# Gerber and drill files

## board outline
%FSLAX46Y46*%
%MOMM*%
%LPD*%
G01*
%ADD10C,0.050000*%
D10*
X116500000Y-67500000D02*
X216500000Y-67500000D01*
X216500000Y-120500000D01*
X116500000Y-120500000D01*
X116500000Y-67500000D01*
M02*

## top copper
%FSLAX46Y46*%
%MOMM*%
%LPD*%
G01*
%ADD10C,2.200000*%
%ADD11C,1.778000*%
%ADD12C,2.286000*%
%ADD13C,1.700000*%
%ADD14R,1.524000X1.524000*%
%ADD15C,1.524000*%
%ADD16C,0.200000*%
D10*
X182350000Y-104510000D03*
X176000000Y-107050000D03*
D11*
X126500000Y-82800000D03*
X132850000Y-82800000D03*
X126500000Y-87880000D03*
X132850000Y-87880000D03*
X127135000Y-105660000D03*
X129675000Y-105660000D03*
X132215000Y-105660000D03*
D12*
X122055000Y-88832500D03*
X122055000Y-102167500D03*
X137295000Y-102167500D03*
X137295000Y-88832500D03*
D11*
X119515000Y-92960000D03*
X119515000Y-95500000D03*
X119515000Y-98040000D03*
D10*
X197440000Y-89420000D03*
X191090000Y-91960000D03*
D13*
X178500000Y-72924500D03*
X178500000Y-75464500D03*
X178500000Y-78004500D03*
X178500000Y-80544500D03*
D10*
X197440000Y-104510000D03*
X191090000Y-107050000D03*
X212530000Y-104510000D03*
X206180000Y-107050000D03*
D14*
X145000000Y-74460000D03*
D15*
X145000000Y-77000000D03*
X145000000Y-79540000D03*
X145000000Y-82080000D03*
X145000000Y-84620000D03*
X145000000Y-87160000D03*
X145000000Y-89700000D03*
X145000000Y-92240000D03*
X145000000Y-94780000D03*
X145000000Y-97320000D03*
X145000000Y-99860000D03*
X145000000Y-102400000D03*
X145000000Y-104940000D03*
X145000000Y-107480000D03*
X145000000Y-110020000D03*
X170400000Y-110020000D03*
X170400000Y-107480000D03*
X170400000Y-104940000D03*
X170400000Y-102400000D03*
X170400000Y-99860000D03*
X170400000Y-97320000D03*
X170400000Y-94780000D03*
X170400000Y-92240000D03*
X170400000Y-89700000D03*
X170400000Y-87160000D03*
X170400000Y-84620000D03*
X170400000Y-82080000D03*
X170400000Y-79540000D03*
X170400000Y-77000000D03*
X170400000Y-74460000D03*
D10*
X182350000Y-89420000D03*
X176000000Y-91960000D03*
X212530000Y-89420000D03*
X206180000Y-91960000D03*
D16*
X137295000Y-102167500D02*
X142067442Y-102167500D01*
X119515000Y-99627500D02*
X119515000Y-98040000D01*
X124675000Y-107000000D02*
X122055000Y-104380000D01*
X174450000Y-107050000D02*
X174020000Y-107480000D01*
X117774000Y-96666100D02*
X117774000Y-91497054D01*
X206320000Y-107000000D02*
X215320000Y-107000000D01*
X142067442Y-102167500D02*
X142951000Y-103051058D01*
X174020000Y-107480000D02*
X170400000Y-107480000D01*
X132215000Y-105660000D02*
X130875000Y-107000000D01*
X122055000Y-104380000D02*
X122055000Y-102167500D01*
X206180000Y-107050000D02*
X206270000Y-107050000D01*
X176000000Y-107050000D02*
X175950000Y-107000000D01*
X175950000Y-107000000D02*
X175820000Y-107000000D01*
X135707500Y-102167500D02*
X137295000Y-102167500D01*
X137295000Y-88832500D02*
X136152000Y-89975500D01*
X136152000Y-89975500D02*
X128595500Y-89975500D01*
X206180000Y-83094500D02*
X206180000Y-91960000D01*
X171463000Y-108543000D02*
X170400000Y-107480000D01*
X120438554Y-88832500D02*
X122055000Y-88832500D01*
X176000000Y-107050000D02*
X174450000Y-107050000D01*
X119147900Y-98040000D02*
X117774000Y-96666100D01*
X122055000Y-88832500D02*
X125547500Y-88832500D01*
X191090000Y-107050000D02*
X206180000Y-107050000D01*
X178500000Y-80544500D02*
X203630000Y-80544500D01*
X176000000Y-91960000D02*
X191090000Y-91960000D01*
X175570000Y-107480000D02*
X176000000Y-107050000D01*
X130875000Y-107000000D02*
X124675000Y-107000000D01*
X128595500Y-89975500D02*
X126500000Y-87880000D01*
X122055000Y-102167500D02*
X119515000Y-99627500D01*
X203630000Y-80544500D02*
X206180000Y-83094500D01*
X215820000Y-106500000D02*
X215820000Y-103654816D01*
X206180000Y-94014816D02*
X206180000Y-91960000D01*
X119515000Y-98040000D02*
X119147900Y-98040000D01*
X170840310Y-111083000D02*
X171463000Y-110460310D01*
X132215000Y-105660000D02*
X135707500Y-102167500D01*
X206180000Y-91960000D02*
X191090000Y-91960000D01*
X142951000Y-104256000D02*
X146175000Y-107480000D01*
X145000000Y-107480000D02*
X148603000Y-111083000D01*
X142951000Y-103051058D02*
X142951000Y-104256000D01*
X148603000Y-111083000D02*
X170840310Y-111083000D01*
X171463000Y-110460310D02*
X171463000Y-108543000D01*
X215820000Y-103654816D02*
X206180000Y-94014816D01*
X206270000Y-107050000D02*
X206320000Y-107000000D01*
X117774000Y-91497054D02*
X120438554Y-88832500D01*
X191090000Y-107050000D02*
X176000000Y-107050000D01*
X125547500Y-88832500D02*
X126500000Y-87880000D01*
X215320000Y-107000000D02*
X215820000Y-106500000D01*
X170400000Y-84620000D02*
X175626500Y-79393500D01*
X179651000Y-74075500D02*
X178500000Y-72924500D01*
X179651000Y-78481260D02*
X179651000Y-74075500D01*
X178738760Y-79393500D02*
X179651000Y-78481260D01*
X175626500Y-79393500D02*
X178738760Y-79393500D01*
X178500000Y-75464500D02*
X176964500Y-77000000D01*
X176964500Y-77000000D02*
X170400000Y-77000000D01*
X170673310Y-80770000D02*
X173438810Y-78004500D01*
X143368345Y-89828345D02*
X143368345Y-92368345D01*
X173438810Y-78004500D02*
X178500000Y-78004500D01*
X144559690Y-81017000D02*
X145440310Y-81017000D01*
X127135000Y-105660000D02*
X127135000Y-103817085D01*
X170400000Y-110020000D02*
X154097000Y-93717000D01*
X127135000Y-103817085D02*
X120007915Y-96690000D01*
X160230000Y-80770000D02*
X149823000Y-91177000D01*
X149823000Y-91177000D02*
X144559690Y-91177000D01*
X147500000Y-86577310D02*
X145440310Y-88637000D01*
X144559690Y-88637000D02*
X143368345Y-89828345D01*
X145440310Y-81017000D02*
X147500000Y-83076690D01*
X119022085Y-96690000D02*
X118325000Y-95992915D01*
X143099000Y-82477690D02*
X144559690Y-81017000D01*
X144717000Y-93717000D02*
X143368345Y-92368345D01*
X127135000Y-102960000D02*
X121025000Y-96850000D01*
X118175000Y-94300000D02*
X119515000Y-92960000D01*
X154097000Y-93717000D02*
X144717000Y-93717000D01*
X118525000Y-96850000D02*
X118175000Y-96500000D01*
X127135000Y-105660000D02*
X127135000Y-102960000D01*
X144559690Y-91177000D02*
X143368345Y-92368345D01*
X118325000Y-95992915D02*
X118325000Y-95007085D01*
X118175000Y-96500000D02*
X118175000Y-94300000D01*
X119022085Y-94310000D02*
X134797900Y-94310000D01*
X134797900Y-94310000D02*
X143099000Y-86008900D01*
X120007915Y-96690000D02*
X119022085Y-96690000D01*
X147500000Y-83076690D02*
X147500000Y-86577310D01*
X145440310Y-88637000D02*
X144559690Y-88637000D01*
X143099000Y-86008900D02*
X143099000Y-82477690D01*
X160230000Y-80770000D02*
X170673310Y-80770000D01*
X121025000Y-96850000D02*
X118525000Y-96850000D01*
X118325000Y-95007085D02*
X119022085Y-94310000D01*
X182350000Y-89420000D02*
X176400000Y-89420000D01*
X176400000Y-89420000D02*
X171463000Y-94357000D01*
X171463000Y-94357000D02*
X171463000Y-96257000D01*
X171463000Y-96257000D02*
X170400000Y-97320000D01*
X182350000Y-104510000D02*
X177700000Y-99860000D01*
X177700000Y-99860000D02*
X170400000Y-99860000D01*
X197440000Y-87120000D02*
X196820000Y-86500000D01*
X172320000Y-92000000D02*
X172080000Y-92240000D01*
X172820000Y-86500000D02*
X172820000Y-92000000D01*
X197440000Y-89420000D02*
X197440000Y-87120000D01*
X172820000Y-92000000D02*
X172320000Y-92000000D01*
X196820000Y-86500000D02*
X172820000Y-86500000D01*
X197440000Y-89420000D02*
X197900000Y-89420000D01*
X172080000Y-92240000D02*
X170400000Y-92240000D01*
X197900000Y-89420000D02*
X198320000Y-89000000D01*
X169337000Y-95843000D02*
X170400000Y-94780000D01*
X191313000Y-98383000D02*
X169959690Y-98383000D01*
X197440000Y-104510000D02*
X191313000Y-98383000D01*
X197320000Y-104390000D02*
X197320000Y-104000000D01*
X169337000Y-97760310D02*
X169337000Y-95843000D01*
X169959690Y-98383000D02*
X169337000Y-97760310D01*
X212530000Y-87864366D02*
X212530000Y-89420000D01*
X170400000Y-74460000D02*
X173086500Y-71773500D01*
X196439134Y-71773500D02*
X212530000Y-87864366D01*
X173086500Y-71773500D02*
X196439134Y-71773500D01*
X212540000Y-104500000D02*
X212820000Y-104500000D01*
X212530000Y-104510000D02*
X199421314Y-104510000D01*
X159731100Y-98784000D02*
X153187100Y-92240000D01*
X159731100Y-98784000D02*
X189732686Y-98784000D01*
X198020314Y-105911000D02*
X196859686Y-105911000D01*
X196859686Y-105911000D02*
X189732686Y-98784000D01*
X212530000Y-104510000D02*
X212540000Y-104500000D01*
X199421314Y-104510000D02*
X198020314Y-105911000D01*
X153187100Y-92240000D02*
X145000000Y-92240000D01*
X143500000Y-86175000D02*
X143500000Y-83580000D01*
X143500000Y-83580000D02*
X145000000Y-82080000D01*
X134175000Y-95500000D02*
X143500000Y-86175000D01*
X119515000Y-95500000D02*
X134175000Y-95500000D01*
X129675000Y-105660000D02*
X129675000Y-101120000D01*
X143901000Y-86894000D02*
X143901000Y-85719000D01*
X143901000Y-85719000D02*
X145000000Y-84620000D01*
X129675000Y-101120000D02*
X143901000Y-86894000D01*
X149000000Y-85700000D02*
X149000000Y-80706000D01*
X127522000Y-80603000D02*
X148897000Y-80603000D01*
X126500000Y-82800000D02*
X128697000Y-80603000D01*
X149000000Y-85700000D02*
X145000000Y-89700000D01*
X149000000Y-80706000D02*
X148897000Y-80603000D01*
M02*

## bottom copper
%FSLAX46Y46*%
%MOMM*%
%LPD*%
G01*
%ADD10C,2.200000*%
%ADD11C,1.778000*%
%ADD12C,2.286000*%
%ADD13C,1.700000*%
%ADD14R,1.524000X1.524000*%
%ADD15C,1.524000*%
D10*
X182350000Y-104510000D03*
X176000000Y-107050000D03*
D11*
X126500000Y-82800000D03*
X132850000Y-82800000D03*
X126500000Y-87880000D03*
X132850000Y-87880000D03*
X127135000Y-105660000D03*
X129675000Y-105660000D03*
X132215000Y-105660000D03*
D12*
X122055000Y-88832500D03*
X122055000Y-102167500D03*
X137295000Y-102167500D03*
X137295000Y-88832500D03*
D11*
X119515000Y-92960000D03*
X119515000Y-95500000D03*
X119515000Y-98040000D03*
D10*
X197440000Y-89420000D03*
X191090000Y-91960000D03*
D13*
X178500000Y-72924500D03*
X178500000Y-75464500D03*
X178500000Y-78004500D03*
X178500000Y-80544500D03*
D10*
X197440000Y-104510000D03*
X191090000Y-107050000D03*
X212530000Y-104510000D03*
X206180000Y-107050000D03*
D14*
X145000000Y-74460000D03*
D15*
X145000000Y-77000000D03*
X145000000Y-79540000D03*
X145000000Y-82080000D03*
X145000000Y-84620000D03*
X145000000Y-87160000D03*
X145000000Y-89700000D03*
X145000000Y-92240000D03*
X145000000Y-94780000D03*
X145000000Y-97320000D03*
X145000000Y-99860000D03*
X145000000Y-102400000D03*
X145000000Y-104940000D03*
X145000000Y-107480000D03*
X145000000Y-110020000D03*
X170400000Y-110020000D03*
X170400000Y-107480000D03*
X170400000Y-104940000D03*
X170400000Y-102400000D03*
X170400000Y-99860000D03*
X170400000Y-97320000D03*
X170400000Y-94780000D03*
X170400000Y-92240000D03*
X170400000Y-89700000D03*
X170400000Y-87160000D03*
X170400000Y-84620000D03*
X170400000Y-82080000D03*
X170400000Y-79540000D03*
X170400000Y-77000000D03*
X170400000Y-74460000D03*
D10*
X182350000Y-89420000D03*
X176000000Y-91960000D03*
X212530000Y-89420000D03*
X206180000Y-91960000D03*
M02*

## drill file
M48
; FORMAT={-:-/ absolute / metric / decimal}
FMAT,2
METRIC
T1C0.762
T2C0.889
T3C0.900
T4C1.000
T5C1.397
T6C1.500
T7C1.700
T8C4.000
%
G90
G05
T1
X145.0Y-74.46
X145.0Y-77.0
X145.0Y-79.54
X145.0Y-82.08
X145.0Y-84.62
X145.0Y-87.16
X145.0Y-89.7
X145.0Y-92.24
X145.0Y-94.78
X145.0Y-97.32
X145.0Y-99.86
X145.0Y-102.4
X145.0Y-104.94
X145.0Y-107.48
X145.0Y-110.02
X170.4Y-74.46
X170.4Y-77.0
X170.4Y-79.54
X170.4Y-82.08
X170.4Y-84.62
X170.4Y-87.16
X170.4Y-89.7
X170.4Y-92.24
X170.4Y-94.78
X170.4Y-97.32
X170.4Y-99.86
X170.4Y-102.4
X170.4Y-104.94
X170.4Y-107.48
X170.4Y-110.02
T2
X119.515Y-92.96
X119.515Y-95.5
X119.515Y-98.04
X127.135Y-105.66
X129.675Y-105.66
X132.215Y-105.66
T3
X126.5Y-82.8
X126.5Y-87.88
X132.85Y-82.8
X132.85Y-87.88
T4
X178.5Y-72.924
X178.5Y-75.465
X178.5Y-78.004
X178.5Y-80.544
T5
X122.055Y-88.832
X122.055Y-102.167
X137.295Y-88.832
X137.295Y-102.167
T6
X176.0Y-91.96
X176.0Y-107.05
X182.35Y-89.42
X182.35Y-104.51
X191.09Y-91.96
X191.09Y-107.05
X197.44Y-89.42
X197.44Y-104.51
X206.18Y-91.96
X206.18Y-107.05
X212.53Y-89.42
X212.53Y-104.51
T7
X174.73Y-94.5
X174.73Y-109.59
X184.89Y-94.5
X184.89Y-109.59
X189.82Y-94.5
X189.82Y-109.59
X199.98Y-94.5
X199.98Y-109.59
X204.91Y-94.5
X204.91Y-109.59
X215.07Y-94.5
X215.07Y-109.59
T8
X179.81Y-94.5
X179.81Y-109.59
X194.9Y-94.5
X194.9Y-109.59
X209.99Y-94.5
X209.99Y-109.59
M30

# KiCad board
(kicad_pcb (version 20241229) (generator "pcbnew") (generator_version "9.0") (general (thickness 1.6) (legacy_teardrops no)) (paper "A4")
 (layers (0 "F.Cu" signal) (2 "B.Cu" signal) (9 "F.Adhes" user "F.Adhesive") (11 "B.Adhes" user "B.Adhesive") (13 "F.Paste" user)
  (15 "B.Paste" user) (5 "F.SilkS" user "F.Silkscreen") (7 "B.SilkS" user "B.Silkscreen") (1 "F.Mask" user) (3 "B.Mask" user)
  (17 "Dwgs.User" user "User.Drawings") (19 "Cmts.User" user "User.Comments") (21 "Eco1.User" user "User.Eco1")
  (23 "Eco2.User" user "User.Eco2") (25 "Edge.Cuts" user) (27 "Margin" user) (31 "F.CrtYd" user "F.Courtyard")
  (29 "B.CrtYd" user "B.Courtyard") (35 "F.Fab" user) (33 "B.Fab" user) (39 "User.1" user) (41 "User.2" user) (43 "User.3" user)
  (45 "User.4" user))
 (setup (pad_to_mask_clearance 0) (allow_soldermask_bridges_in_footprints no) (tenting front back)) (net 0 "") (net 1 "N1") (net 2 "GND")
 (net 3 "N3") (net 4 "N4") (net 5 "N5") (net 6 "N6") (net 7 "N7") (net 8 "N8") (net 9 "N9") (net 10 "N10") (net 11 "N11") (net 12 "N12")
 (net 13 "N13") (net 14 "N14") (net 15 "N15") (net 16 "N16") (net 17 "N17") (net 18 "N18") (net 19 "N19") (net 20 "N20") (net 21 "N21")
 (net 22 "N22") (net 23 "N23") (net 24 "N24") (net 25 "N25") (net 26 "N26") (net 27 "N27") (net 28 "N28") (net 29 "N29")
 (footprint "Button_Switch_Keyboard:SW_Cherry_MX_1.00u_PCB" (layer "F.Cu") (at 182.35 104.51)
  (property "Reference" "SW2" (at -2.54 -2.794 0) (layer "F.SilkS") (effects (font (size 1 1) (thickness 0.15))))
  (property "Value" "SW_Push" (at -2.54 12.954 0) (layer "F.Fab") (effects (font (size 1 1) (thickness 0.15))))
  (pad "" np_thru_hole circle (at -7.62 5.08) (size 1.7 1.7) (drill 1.7) (layers "*.Cu" "*.Mask"))
  (pad "" np_thru_hole circle (at -2.54 5.08) (size 4 4) (drill 4) (layers "*.Cu" "*.Mask"))
  (pad "" np_thru_hole circle (at 2.54 5.08) (size 1.7 1.7) (drill 1.7) (layers "*.Cu" "*.Mask"))
  (pad "1" thru_hole circle (at 0 0) (size 2.2 2.2) (drill 1.5) (layers "*.Cu" "*.Mask") (remove_unused_layers no) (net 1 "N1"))
  (pad "2" thru_hole circle (at -6.35 2.54) (size 2.2 2.2) (drill 1.5) (layers "*.Cu" "*.Mask") (remove_unused_layers no) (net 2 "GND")))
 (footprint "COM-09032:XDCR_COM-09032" (layer "F.Cu") (at 129.675 95.5)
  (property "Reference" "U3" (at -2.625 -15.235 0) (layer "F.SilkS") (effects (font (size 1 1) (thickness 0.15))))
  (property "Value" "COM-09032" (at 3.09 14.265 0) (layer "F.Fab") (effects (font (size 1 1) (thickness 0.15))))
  (pad "B1A" thru_hole circle (at -3.175 -12.7) (size 1.778 1.778) (drill 0.9) (layers "*.Cu" "*.Mask") (remove_unused_layers no)
   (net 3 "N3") (solder_mask_margin 0.102))
  (pad "B1B" thru_hole circle (at 3.175 -12.7) (size 1.778 1.778) (drill 0.9) (layers "*.Cu" "*.Mask") (remove_unused_layers no)
   (solder_mask_margin 0.102))
  (pad "B2A" thru_hole circle (at -3.175 -7.62) (size 1.778 1.778) (drill 0.9) (layers "*.Cu" "*.Mask") (remove_unused_layers no)
   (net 2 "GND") (solder_mask_margin 0.102))
  (pad "B2B" thru_hole circle (at 3.175 -7.62) (size 1.778 1.778) (drill 0.9) (layers "*.Cu" "*.Mask") (remove_unused_layers no)
   (solder_mask_margin 0.102))
  (pad "H1" thru_hole circle (at -2.54 10.16) (size 1.778 1.778) (drill 0.889) (layers "*.Cu" "*.Mask") (remove_unused_layers no)
   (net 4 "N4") (solder_mask_margin 0.102))
  (pad "H2" thru_hole circle (at 0 10.16) (size 1.778 1.778) (drill 0.889) (layers "*.Cu" "*.Mask") (remove_unused_layers no) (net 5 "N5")
   (solder_mask_margin 0.102))
  (pad "H3" thru_hole circle (at 2.54 10.16) (size 1.778 1.778) (drill 0.889) (layers "*.Cu" "*.Mask") (remove_unused_layers no)
   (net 2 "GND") (solder_mask_margin 0.102))
  (pad "S1" thru_hole circle (at -7.62 -6.6675) (size 2.286 2.286) (drill 1.397) (layers "*.Cu" "*.Mask") (remove_unused_layers no)
   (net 2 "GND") (solder_mask_margin 0.102))
  (pad "S2" thru_hole circle (at -7.62 6.6675) (size 2.286 2.286) (drill 1.397) (layers "*.Cu" "*.Mask") (remove_unused_layers no)
   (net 2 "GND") (solder_mask_margin 0.102))
  (pad "S3" thru_hole circle (at 7.62 6.6675) (size 2.286 2.286) (drill 1.397) (layers "*.Cu" "*.Mask") (remove_unused_layers no)
   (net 2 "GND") (solder_mask_margin 0.102))
  (pad "S4" thru_hole circle (at 7.62 -6.6675) (size 2.286 2.286) (drill 1.397) (layers "*.Cu" "*.Mask") (remove_unused_layers no)
   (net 2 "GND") (solder_mask_margin 0.102))
  (pad "V1" thru_hole circle (at -10.16 -2.54) (size 1.778 1.778) (drill 0.889) (layers "*.Cu" "*.Mask") (remove_unused_layers no)
   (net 4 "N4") (solder_mask_margin 0.102))
  (pad "V2" thru_hole circle (at -10.16 0) (size 1.778 1.778) (drill 0.889) (layers "*.Cu" "*.Mask") (remove_unused_layers no) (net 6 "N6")
   (solder_mask_margin 0.102))
  (pad "V3" thru_hole circle (at -10.16 2.54) (size 1.778 1.778) (drill 0.889) (layers "*.Cu" "*.Mask") (remove_unused_layers no)
   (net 2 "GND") (solder_mask_margin 0.102)))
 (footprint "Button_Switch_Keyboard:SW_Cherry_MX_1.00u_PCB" (layer "F.Cu") (at 197.44 89.42)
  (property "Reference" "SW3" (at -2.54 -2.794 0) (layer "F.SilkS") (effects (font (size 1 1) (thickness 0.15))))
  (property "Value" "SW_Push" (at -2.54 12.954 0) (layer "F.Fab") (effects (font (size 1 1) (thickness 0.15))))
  (pad "" np_thru_hole circle (at -7.62 5.08) (size 1.7 1.7) (drill 1.7) (layers "*.Cu" "*.Mask"))
  (pad "" np_thru_hole circle (at -2.54 5.08) (size 4 4) (drill 4) (layers "*.Cu" "*.Mask"))
  (pad "" np_thru_hole circle (at 2.54 5.08) (size 1.7 1.7) (drill 1.7) (layers "*.Cu" "*.Mask"))
  (pad "1" thru_hole circle (at 0 0) (size 2.2 2.2) (drill 1.5) (layers "*.Cu" "*.Mask") (remove_unused_layers no) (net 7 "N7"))
  (pad "2" thru_hole circle (at -6.35 2.54) (size 2.2 2.2) (drill 1.5) (layers "*.Cu" "*.Mask") (remove_unused_layers no) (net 2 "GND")))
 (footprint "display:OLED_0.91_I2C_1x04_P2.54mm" (layer "F.Cu") (at 178.5 72.9245)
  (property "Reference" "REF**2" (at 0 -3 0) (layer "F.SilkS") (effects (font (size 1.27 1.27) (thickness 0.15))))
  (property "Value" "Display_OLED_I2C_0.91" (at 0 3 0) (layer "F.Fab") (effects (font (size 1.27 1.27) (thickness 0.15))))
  (pad "1" thru_hole circle (at 0 0) (size 1.7 1.7) (drill 1) (layers "*.Cu" "*.Mask") (remove_unused_layers no) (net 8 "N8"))
  (pad "2" thru_hole circle (at 0 2.54) (size 1.7 1.7) (drill 1) (layers "*.Cu" "*.Mask") (remove_unused_layers no) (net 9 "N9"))
  (pad "3" thru_hole circle (at 0 5.08) (size 1.7 1.7) (drill 1) (layers "*.Cu" "*.Mask") (remove_unused_layers no) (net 4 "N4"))
  (pad "4" thru_hole circle (at 0 7.62) (size 1.7 1.7) (drill 1) (layers "*.Cu" "*.Mask") (remove_unused_layers no) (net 2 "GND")))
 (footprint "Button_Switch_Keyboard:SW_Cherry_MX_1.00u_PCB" (layer "F.Cu") (at 197.44 104.51)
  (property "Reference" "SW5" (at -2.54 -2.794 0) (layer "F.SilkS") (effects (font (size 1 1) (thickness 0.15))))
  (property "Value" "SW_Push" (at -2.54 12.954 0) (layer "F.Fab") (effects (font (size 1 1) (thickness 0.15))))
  (pad "" np_thru_hole circle (at -7.62 5.08) (size 1.7 1.7) (drill 1.7) (layers "*.Cu" "*.Mask"))
  (pad "" np_thru_hole circle (at -2.54 5.08) (size 4 4) (drill 4) (layers "*.Cu" "*.Mask"))
  (pad "" np_thru_hole circle (at 2.54 5.08) (size 1.7 1.7) (drill 1.7) (layers "*.Cu" "*.Mask"))
  (pad "1" thru_hole circle (at 0 0) (size 2.2 2.2) (drill 1.5) (layers "*.Cu" "*.Mask") (remove_unused_layers no) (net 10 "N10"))
  (pad "2" thru_hole circle (at -6.35 2.54) (size 2.2 2.2) (drill 1.5) (layers "*.Cu" "*.Mask") (remove_unused_layers no) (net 2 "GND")))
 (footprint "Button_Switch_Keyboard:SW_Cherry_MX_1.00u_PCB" (layer "F.Cu") (at 212.53 104.51)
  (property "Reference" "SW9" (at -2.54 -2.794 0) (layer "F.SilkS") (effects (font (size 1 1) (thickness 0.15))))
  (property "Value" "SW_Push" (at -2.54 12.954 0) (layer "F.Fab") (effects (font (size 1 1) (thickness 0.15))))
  (pad "" np_thru_hole circle (at -7.62 5.08) (size 1.7 1.7) (drill 1.7) (layers "*.Cu" "*.Mask"))
  (pad "" np_thru_hole circle (at -2.54 5.08) (size 4 4) (drill 4) (layers "*.Cu" "*.Mask"))
  (pad "" np_thru_hole circle (at 2.54 5.08) (size 1.7 1.7) (drill 1.7) (layers "*.Cu" "*.Mask"))
  (pad "1" thru_hole circle (at 0 0) (size 2.2 2.2) (drill 1.5) (layers "*.Cu" "*.Mask") (remove_unused_layers no) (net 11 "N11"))
  (pad "2" thru_hole circle (at -6.35 2.54) (size 2.2 2.2) (drill 1.5) (layers "*.Cu" "*.Mask") (remove_unused_layers no) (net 2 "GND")))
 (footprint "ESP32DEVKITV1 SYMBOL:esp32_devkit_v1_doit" (layer "F.Cu") (at 157.7 74.46)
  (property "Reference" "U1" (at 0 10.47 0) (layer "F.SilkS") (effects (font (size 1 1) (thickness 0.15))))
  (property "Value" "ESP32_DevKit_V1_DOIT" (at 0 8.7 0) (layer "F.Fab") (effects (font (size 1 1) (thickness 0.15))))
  (pad "1" thru_hole rect (at -12.7 0) (size 1.524 1.524) (drill 0.762) (layers "*.Cu" "*.Mask") (remove_unused_layers no) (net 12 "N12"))
  (pad "2" thru_hole circle (at -12.7 2.54) (size 1.524 1.524) (drill 0.762) (layers "*.Cu" "*.Mask") (remove_unused_layers no)
   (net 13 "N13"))
  (pad "3" thru_hole circle (at -12.7 5.08) (size 1.524 1.524) (drill 0.762) (layers "*.Cu" "*.Mask") (remove_unused_layers no)
   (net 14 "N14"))
  (pad "4" thru_hole circle (at -12.7 7.62) (size 1.524 1.524) (drill 0.762) (layers "*.Cu" "*.Mask") (remove_unused_layers no) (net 6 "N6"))
  (pad "5" thru_hole circle (at -12.7 10.16) (size 1.524 1.524) (drill 0.762) (layers "*.Cu" "*.Mask") (remove_unused_layers no)
   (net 5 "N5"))
  (pad "6" thru_hole circle (at -12.7 12.7) (size 1.524 1.524) (drill 0.762) (layers "*.Cu" "*.Mask") (remove_unused_layers no)
   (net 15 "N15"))
  (pad "7" thru_hole circle (at -12.7 15.24) (size 1.524 1.524) (drill 0.762) (layers "*.Cu" "*.Mask") (remove_unused_layers no)
   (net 3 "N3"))
  (pad "8" thru_hole circle (at -12.7 17.78) (size 1.524 1.524) (drill 0.762) (layers "*.Cu" "*.Mask") (remove_unused_layers no)
   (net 11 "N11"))
  (pad "9" thru_hole circle (at -12.7 20.32) (size 1.524 1.524) (drill 0.762) (layers "*.Cu" "*.Mask") (remove_unused_layers no)
   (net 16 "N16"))
  (pad "10" thru_hole circle (at -12.7 22.86) (size 1.524 1.524) (drill 0.762) (layers "*.Cu" "*.Mask") (remove_unused_layers no)
   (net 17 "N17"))
  (pad "11" thru_hole circle (at -12.7 25.4) (size 1.524 1.524) (drill 0.762) (layers "*.Cu" "*.Mask") (remove_unused_layers no)
   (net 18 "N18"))
  (pad "12" thru_hole circle (at -12.7 27.94) (size 1.524 1.524) (drill 0.762) (layers "*.Cu" "*.Mask") (remove_unused_layers no)
   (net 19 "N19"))
  (pad "13" thru_hole circle (at -12.7 30.48) (size 1.524 1.524) (drill 0.762) (layers "*.Cu" "*.Mask") (remove_unused_layers no)
   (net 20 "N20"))
  (pad "14" thru_hole circle (at -12.7 33.02) (size 1.524 1.524) (drill 0.762) (layers "*.Cu" "*.Mask") (remove_unused_layers no)
   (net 2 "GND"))
  (pad "15" thru_hole circle (at -12.7 35.56) (size 1.524 1.524) (drill 0.762) (layers "*.Cu" "*.Mask") (remove_unused_layers no)
   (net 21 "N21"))
  (pad "16" thru_hole circle (at 12.7 35.56) (size 1.524 1.524) (drill 0.762) (layers "*.Cu" "*.Mask") (remove_unused_layers no)
   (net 4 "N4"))
  (pad "17" thru_hole circle (at 12.7 33.02) (size 1.524 1.524) (drill 0.762) (layers "*.Cu" "*.Mask") (remove_unused_layers no)
   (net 2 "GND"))
  (pad "18" thru_hole circle (at 12.7 30.48) (size 1.524 1.524) (drill 0.762) (layers "*.Cu" "*.Mask") (remove_unused_layers no)
   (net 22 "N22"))
  (pad "19" thru_hole circle (at 12.7 27.94) (size 1.524 1.524) (drill 0.762) (layers "*.Cu" "*.Mask") (remove_unused_layers no)
   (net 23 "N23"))
  (pad "20" thru_hole circle (at 12.7 25.4) (size 1.524 1.524) (drill 0.762) (layers "*.Cu" "*.Mask") (remove_unused_layers no) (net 1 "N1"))
  (pad "21" thru_hole circle (at 12.7 22.86) (size 1.524 1.524) (drill 0.762) (layers "*.Cu" "*.Mask") (remove_unused_layers no)
   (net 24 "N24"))
  (pad "22" thru_hole circle (at 12.7 20.32) (size 1.524 1.524) (drill 0.762) (layers "*.Cu" "*.Mask") (remove_unused_layers no)
   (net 10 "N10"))
  (pad "23" thru_hole circle (at 12.7 17.78) (size 1.524 1.524) (drill 0.762) (layers "*.Cu" "*.Mask") (remove_unused_layers no)
   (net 7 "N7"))
  (pad "24" thru_hole circle (at 12.7 15.24) (size 1.524 1.524) (drill 0.762) (layers "*.Cu" "*.Mask") (remove_unused_layers no)
   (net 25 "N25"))
  (pad "25" thru_hole circle (at 12.7 12.7) (size 1.524 1.524) (drill 0.762) (layers "*.Cu" "*.Mask") (remove_unused_layers no)
   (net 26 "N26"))
  (pad "26" thru_hole circle (at 12.7 10.16) (size 1.524 1.524) (drill 0.762) (layers "*.Cu" "*.Mask") (remove_unused_layers no)
   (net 8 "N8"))
  (pad "27" thru_hole circle (at 12.7 7.62) (size 1.524 1.524) (drill 0.762) (layers "*.Cu" "*.Mask") (remove_unused_layers no)
   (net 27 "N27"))
  (pad "28" thru_hole circle (at 12.7 5.08) (size 1.524 1.524) (drill 0.762) (layers "*.Cu" "*.Mask") (remove_unused_layers no)
   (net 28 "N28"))
  (pad "29" thru_hole circle (at 12.7 2.54) (size 1.524 1.524) (drill 0.762) (layers "*.Cu" "*.Mask") (remove_unused_layers no) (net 9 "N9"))
  (pad "30" thru_hole circle (at 12.7 0) (size 1.524 1.524) (drill 0.762) (layers "*.Cu" "*.Mask") (remove_unused_layers no) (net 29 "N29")))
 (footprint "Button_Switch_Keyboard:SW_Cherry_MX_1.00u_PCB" (layer "F.Cu") (at 182.35 89.42)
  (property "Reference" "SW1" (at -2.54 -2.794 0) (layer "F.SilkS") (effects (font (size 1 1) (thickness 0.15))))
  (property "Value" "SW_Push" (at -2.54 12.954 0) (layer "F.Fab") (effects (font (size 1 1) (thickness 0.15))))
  (pad "" np_thru_hole circle (at -7.62 5.08) (size 1.7 1.7) (drill 1.7) (layers "*.Cu" "*.Mask"))
  (pad "" np_thru_hole circle (at -2.54 5.08) (size 4 4) (drill 4) (layers "*.Cu" "*.Mask"))
  (pad "" np_thru_hole circle (at 2.54 5.08) (size 1.7 1.7) (drill 1.7) (layers "*.Cu" "*.Mask"))
  (pad "1" thru_hole circle (at 0 0) (size 2.2 2.2) (drill 1.5) (layers "*.Cu" "*.Mask") (remove_unused_layers no) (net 24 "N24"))
  (pad "2" thru_hole circle (at -6.35 2.54) (size 2.2 2.2) (drill 1.5) (layers "*.Cu" "*.Mask") (remove_unused_layers no) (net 2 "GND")))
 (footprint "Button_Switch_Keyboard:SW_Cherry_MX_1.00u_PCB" (layer "F.Cu") (at 212.53 89.42)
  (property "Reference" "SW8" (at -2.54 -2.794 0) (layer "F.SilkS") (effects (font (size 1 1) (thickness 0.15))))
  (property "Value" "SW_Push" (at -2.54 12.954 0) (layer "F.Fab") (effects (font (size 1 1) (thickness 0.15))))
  (pad "" np_thru_hole circle (at -7.62 5.08) (size 1.7 1.7) (drill 1.7) (layers "*.Cu" "*.Mask"))
  (pad "" np_thru_hole circle (at -2.54 5.08) (size 4 4) (drill 4) (layers "*.Cu" "*.Mask"))
  (pad "" np_thru_hole circle (at 2.54 5.08) (size 1.7 1.7) (drill 1.7) (layers "*.Cu" "*.Mask"))
  (pad "1" thru_hole circle (at 0 0) (size 2.2 2.2) (drill 1.5) (layers "*.Cu" "*.Mask") (remove_unused_layers no) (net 29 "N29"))
  (pad "2" thru_hole circle (at -6.35 2.54) (size 2.2 2.2) (drill 1.5) (layers "*.Cu" "*.Mask") (remove_unused_layers no) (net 2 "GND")))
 (gr_rect (start 116.5 67.5) (end 216.5 120.5) (stroke (width 0.05) (type default)) (fill no) (layer "Edge.Cuts"))
 (segment (start 137.295 102.1675) (end 142.067442 102.1675) (width 0.2) (layer "F.Cu") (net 2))
 (segment (start 119.515 99.6275) (end 119.515 98.04) (width 0.2) (layer "F.Cu") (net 2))
 (segment (start 124.675 107) (end 122.055 104.38) (width 0.2) (layer "F.Cu") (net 2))
 (segment (start 174.45 107.05) (end 174.02 107.48) (width 0.2) (layer "F.Cu") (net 2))
 (segment (start 117.774 96.6661) (end 117.774 91.497054) (width 0.2) (layer "F.Cu") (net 2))
 (segment (start 206.32 107) (end 215.32 107) (width 0.2) (layer "F.Cu") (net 2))
 (segment (start 142.067442 102.1675) (end 142.951 103.051058) (width 0.2) (layer "F.Cu") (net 2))
 (segment (start 174.02 107.48) (end 170.4 107.48) (width 0.2) (layer "F.Cu") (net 2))
 (segment (start 132.215 105.66) (end 130.875 107) (width 0.2) (layer "F.Cu") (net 2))
 (segment (start 122.055 104.38) (end 122.055 102.1675) (width 0.2) (layer "F.Cu") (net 2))
 (segment (start 206.18 107.05) (end 206.27 107.05) (width 0.2) (layer "F.Cu") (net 2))
 (segment (start 176 107.05) (end 175.95 107) (width 0.2) (layer "F.Cu") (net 2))
 (segment (start 175.95 107) (end 175.82 107) (width 0.2) (layer "F.Cu") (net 2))
 (segment (start 135.7075 102.1675) (end 137.295 102.1675) (width 0.2) (layer "F.Cu") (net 2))
 (segment (start 137.295 88.8325) (end 136.152 89.9755) (width 0.2) (layer "F.Cu") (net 2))
 (segment (start 136.152 89.9755) (end 128.5955 89.9755) (width 0.2) (layer "F.Cu") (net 2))
 (segment (start 206.18 83.0945) (end 206.18 91.96) (width 0.2) (layer "F.Cu") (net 2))
 (segment (start 171.463 108.543) (end 170.4 107.48) (width 0.2) (layer "F.Cu") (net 2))
 (segment (start 120.438554 88.8325) (end 122.055 88.8325) (width 0.2) (layer "F.Cu") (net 2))
 (segment (start 176 107.05) (end 174.45 107.05) (width 0.2) (layer "F.Cu") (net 2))
 (segment (start 119.1479 98.04) (end 117.774 96.6661) (width 0.2) (layer "F.Cu") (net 2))
 (segment (start 122.055 88.8325) (end 125.5475 88.8325) (width 0.2) (layer "F.Cu") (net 2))
 (segment (start 191.09 107.05) (end 206.18 107.05) (width 0.2) (layer "F.Cu") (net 2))
 (segment (start 178.5 80.5445) (end 203.63 80.5445) (width 0.2) (layer "F.Cu") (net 2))
 (segment (start 176 91.96) (end 191.09 91.96) (width 0.2) (layer "F.Cu") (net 2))
 (segment (start 175.57 107.48) (end 176 107.05) (width 0.2) (layer "F.Cu") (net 2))
 (segment (start 130.875 107) (end 124.675 107) (width 0.2) (layer "F.Cu") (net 2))
 (segment (start 128.5955 89.9755) (end 126.5 87.88) (width 0.2) (layer "F.Cu") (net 2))
 (segment (start 122.055 102.1675) (end 119.515 99.6275) (width 0.2) (layer "F.Cu") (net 2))
 (segment (start 203.63 80.5445) (end 206.18 83.0945) (width 0.2) (layer "F.Cu") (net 2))
 (segment (start 215.82 106.5) (end 215.82 103.654816) (width 0.2) (layer "F.Cu") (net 2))
 (segment (start 206.18 94.014816) (end 206.18 91.96) (width 0.2) (layer "F.Cu") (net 2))
 (segment (start 119.515 98.04) (end 119.1479 98.04) (width 0.2) (layer "F.Cu") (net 2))
 (segment (start 170.84031 111.083) (end 171.463 110.46031) (width 0.2) (layer "F.Cu") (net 2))
 (segment (start 132.215 105.66) (end 135.7075 102.1675) (width 0.2) (layer "F.Cu") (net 2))
 (segment (start 206.18 91.96) (end 191.09 91.96) (width 0.2) (layer "F.Cu") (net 2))
 (segment (start 142.951 104.256) (end 146.175 107.48) (width 0.2) (layer "F.Cu") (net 2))
 (segment (start 145 107.48) (end 148.603 111.083) (width 0.2) (layer "F.Cu") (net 2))
 (segment (start 142.951 103.051058) (end 142.951 104.256) (width 0.2) (layer "F.Cu") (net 2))
 (segment (start 148.603 111.083) (end 170.84031 111.083) (width 0.2) (layer "F.Cu") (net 2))
 (segment (start 171.463 110.46031) (end 171.463 108.543) (width 0.2) (layer "F.Cu") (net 2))
 (segment (start 215.82 103.654816) (end 206.18 94.014816) (width 0.2) (layer "F.Cu") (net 2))
 (segment (start 206.27 107.05) (end 206.32 107) (width 0.2) (layer "F.Cu") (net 2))
 (segment (start 117.774 91.497054) (end 120.438554 88.8325) (width 0.2) (layer "F.Cu") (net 2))
 (segment (start 191.09 107.05) (end 176 107.05) (width 0.2) (layer "F.Cu") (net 2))
 (segment (start 125.5475 88.8325) (end 126.5 87.88) (width 0.2) (layer "F.Cu") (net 2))
 (segment (start 215.32 107) (end 215.82 106.5) (width 0.2) (layer "F.Cu") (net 2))
 (segment (start 170.4 84.62) (end 175.6265 79.3935) (width 0.2) (layer "F.Cu") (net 8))
 (segment (start 179.651 74.0755) (end 178.5 72.9245) (width 0.2) (layer "F.Cu") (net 8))
 (segment (start 179.651 78.48126) (end 179.651 74.0755) (width 0.2) (layer "F.Cu") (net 8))
 (segment (start 178.73876 79.3935) (end 179.651 78.48126) (width 0.2) (layer "F.Cu") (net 8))
 (segment (start 175.6265 79.3935) (end 178.73876 79.3935) (width 0.2) (layer "F.Cu") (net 8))
 (segment (start 178.5 75.4645) (end 176.9645 77) (width 0.2) (layer "F.Cu") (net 9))
 (segment (start 176.9645 77) (end 170.4 77) (width 0.2) (layer "F.Cu") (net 9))
 (segment (start 170.67331 80.77) (end 173.43881 78.0045) (width 0.2) (layer "F.Cu") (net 4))
 (segment (start 143.368345 89.828345) (end 143.368345 92.368345) (width 0.2) (layer "F.Cu") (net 4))
 (segment (start 173.43881 78.0045) (end 178.5 78.0045) (width 0.2) (layer "F.Cu") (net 4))
 (segment (start 144.55969 81.017) (end 145.44031 81.017) (width 0.2) (layer "F.Cu") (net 4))
 (segment (start 127.135 105.66) (end 127.135 103.817085) (width 0.2) (layer "F.Cu") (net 4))
 (segment (start 170.4 110.02) (end 154.097 93.717) (width 0.2) (layer "F.Cu") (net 4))
 (segment (start 127.135 103.817085) (end 120.007915 96.69) (width 0.2) (layer "F.Cu") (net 4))
 (segment (start 160.23 80.77) (end 149.823 91.177) (width 0.2) (layer "F.Cu") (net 4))
 (segment (start 149.823 91.177) (end 144.55969 91.177) (width 0.2) (layer "F.Cu") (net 4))
 (segment (start 147.5 86.57731) (end 145.44031 88.637) (width 0.2) (layer "F.Cu") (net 4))
 (segment (start 144.55969 88.637) (end 143.368345 89.828345) (width 0.2) (layer "F.Cu") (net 4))
 (segment (start 145.44031 81.017) (end 147.5 83.07669) (width 0.2) (layer "F.Cu") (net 4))
 (segment (start 119.022085 96.69) (end 118.325 95.992915) (width 0.2) (layer "F.Cu") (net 4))
 (segment (start 143.099 82.47769) (end 144.55969 81.017) (width 0.2) (layer "F.Cu") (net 4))
 (segment (start 144.717 93.717) (end 143.368345 92.368345) (width 0.2) (layer "F.Cu") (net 4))
 (segment (start 127.135 102.96) (end 121.025 96.85) (width 0.2) (layer "F.Cu") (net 4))
 (segment (start 118.175 94.3) (end 119.515 92.96) (width 0.2) (layer "F.Cu") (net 4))
 (segment (start 154.097 93.717) (end 144.717 93.717) (width 0.2) (layer "F.Cu") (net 4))
 (segment (start 118.525 96.85) (end 118.175 96.5) (width 0.2) (layer "F.Cu") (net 4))
 (segment (start 127.135 105.66) (end 127.135 102.96) (width 0.2) (layer "F.Cu") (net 4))
 (segment (start 144.55969 91.177) (end 143.368345 92.368345) (width 0.2) (layer "F.Cu") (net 4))
 (segment (start 118.325 95.992915) (end 118.325 95.007085) (width 0.2) (layer "F.Cu") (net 4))
 (segment (start 118.175 96.5) (end 118.175 94.3) (width 0.2) (layer "F.Cu") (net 4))
 (segment (start 119.022085 94.31) (end 134.7979 94.31) (width 0.2) (layer "F.Cu") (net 4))
 (segment (start 134.7979 94.31) (end 143.099 86.0089) (width 0.2) (layer "F.Cu") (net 4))
 (segment (start 120.007915 96.69) (end 119.022085 96.69) (width 0.2) (layer "F.Cu") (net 4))
 (segment (start 147.5 83.07669) (end 147.5 86.57731) (width 0.2) (layer "F.Cu") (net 4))
 (segment (start 145.44031 88.637) (end 144.55969 88.637) (width 0.2) (layer "F.Cu") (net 4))
 (segment (start 143.099 86.0089) (end 143.099 82.47769) (width 0.2) (layer "F.Cu") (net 4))
 (segment (start 160.23 80.77) (end 170.67331 80.77) (width 0.2) (layer "F.Cu") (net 4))
 (segment (start 121.025 96.85) (end 118.525 96.85) (width 0.2) (layer "F.Cu") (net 4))
 (segment (start 118.325 95.007085) (end 119.022085 94.31) (width 0.2) (layer "F.Cu") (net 4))
 (segment (start 182.35 89.42) (end 176.4 89.42) (width 0.2) (layer "F.Cu") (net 24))
 (segment (start 176.4 89.42) (end 171.463 94.357) (width 0.2) (layer "F.Cu") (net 24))
 (segment (start 171.463 94.357) (end 171.463 96.257) (width 0.2) (layer "F.Cu") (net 24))
 (segment (start 171.463 96.257) (end 170.4 97.32) (width 0.2) (layer "F.Cu") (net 24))
 (segment (start 182.35 104.51) (end 177.7 99.86) (width 0.2) (layer "F.Cu") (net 1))
 (segment (start 177.7 99.86) (end 170.4 99.86) (width 0.2) (layer "F.Cu") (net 1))
 (segment (start 197.44 87.12) (end 196.82 86.5) (width 0.2) (layer "F.Cu") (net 7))
 (segment (start 172.32 92) (end 172.08 92.24) (width 0.2) (layer "F.Cu") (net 7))
 (segment (start 172.82 86.5) (end 172.82 92) (width 0.2) (layer "F.Cu") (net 7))
 (segment (start 197.44 89.42) (end 197.44 87.12) (width 0.2) (layer "F.Cu") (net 7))
 (segment (start 172.82 92) (end 172.32 92) (width 0.2) (layer "F.Cu") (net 7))
 (segment (start 196.82 86.5) (end 172.82 86.5) (width 0.2) (layer "F.Cu") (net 7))
 (segment (start 197.44 89.42) (end 197.9 89.42) (width 0.2) (layer "F.Cu") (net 7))
 (segment (start 172.08 92.24) (end 170.4 92.24) (width 0.2) (layer "F.Cu") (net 7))
 (segment (start 197.9 89.42) (end 198.32 89) (width 0.2) (layer "F.Cu") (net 7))
 (segment (start 169.337 95.843) (end 170.4 94.78) (width 0.2) (layer "F.Cu") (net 10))
 (segment (start 191.313 98.383) (end 169.95969 98.383) (width 0.2) (layer "F.Cu") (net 10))
 (segment (start 197.44 104.51) (end 191.313 98.383) (width 0.2) (layer "F.Cu") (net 10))
 (segment (start 197.32 104.39) (end 197.32 104) (width 0.2) (layer "F.Cu") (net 10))
 (segment (start 169.337 97.76031) (end 169.337 95.843) (width 0.2) (layer "F.Cu") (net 10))
 (segment (start 169.95969 98.383) (end 169.337 97.76031) (width 0.2) (layer "F.Cu") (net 10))
 (segment (start 212.53 87.864366) (end 212.53 89.42) (width 0.2) (layer "F.Cu") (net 29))
 (segment (start 170.4 74.46) (end 173.0865 71.7735) (width 0.2) (layer "F.Cu") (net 29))
 (segment (start 196.439134 71.7735) (end 212.53 87.864366) (width 0.2) (layer "F.Cu") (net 29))
 (segment (start 173.0865 71.7735) (end 196.439134 71.7735) (width 0.2) (layer "F.Cu") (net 29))
 (segment (start 212.54 104.5) (end 212.82 104.5) (width 0.2) (layer "F.Cu") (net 11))
 (segment (start 212.53 104.51) (end 199.421314 104.51) (width 0.2) (layer "F.Cu") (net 11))
 (segment (start 159.7311 98.784) (end 153.1871 92.24) (width 0.2) (layer "F.Cu") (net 11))
 (segment (start 159.7311 98.784) (end 189.732686 98.784) (width 0.2) (layer "F.Cu") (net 11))
 (segment (start 198.020314 105.911) (end 196.859686 105.911) (width 0.2) (layer "F.Cu") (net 11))
 (segment (start 196.859686 105.911) (end 189.732686 98.784) (width 0.2) (layer "F.Cu") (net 11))
 (segment (start 212.53 104.51) (end 212.54 104.5) (width 0.2) (layer "F.Cu") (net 11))
 (segment (start 199.421314 104.51) (end 198.020314 105.911) (width 0.2) (layer "F.Cu") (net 11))
 (segment (start 153.1871 92.24) (end 145 92.24) (width 0.2) (layer "F.Cu") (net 11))
 (segment (start 143.5 86.175) (end 143.5 83.58) (width 0.2) (layer "F.Cu") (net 6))
 (segment (start 143.5 83.58) (end 145 82.08) (width 0.2) (layer "F.Cu") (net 6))
 (segment (start 134.175 95.5) (end 143.5 86.175) (width 0.2) (layer "F.Cu") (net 6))
 (segment (start 119.515 95.5) (end 134.175 95.5) (width 0.2) (layer "F.Cu") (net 6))
 (segment (start 129.675 105.66) (end 129.675 101.12) (width 0.2) (layer "F.Cu") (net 5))
 (segment (start 143.901 86.894) (end 143.901 85.719) (width 0.2) (layer "F.Cu") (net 5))
 (segment (start 143.901 85.719) (end 145 84.62) (width 0.2) (layer "F.Cu") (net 5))
 (segment (start 129.675 101.12) (end 143.901 86.894) (width 0.2) (layer "F.Cu") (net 5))
 (segment (start 149 85.7) (end 149 80.706) (width 0.2) (layer "F.Cu") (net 3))
 (segment (start 127.522 80.603) (end 148.897 80.603) (width 0.2) (layer "F.Cu") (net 3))
 (segment (start 126.5 82.8) (end 128.697 80.603) (width 0.2) (layer "F.Cu") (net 3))
 (segment (start 149 85.7) (end 145 89.7) (width 0.2) (layer "F.Cu") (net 3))
 (segment (start 149 80.706) (end 148.897 80.603) (width 0.2) (layer "F.Cu") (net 3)))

